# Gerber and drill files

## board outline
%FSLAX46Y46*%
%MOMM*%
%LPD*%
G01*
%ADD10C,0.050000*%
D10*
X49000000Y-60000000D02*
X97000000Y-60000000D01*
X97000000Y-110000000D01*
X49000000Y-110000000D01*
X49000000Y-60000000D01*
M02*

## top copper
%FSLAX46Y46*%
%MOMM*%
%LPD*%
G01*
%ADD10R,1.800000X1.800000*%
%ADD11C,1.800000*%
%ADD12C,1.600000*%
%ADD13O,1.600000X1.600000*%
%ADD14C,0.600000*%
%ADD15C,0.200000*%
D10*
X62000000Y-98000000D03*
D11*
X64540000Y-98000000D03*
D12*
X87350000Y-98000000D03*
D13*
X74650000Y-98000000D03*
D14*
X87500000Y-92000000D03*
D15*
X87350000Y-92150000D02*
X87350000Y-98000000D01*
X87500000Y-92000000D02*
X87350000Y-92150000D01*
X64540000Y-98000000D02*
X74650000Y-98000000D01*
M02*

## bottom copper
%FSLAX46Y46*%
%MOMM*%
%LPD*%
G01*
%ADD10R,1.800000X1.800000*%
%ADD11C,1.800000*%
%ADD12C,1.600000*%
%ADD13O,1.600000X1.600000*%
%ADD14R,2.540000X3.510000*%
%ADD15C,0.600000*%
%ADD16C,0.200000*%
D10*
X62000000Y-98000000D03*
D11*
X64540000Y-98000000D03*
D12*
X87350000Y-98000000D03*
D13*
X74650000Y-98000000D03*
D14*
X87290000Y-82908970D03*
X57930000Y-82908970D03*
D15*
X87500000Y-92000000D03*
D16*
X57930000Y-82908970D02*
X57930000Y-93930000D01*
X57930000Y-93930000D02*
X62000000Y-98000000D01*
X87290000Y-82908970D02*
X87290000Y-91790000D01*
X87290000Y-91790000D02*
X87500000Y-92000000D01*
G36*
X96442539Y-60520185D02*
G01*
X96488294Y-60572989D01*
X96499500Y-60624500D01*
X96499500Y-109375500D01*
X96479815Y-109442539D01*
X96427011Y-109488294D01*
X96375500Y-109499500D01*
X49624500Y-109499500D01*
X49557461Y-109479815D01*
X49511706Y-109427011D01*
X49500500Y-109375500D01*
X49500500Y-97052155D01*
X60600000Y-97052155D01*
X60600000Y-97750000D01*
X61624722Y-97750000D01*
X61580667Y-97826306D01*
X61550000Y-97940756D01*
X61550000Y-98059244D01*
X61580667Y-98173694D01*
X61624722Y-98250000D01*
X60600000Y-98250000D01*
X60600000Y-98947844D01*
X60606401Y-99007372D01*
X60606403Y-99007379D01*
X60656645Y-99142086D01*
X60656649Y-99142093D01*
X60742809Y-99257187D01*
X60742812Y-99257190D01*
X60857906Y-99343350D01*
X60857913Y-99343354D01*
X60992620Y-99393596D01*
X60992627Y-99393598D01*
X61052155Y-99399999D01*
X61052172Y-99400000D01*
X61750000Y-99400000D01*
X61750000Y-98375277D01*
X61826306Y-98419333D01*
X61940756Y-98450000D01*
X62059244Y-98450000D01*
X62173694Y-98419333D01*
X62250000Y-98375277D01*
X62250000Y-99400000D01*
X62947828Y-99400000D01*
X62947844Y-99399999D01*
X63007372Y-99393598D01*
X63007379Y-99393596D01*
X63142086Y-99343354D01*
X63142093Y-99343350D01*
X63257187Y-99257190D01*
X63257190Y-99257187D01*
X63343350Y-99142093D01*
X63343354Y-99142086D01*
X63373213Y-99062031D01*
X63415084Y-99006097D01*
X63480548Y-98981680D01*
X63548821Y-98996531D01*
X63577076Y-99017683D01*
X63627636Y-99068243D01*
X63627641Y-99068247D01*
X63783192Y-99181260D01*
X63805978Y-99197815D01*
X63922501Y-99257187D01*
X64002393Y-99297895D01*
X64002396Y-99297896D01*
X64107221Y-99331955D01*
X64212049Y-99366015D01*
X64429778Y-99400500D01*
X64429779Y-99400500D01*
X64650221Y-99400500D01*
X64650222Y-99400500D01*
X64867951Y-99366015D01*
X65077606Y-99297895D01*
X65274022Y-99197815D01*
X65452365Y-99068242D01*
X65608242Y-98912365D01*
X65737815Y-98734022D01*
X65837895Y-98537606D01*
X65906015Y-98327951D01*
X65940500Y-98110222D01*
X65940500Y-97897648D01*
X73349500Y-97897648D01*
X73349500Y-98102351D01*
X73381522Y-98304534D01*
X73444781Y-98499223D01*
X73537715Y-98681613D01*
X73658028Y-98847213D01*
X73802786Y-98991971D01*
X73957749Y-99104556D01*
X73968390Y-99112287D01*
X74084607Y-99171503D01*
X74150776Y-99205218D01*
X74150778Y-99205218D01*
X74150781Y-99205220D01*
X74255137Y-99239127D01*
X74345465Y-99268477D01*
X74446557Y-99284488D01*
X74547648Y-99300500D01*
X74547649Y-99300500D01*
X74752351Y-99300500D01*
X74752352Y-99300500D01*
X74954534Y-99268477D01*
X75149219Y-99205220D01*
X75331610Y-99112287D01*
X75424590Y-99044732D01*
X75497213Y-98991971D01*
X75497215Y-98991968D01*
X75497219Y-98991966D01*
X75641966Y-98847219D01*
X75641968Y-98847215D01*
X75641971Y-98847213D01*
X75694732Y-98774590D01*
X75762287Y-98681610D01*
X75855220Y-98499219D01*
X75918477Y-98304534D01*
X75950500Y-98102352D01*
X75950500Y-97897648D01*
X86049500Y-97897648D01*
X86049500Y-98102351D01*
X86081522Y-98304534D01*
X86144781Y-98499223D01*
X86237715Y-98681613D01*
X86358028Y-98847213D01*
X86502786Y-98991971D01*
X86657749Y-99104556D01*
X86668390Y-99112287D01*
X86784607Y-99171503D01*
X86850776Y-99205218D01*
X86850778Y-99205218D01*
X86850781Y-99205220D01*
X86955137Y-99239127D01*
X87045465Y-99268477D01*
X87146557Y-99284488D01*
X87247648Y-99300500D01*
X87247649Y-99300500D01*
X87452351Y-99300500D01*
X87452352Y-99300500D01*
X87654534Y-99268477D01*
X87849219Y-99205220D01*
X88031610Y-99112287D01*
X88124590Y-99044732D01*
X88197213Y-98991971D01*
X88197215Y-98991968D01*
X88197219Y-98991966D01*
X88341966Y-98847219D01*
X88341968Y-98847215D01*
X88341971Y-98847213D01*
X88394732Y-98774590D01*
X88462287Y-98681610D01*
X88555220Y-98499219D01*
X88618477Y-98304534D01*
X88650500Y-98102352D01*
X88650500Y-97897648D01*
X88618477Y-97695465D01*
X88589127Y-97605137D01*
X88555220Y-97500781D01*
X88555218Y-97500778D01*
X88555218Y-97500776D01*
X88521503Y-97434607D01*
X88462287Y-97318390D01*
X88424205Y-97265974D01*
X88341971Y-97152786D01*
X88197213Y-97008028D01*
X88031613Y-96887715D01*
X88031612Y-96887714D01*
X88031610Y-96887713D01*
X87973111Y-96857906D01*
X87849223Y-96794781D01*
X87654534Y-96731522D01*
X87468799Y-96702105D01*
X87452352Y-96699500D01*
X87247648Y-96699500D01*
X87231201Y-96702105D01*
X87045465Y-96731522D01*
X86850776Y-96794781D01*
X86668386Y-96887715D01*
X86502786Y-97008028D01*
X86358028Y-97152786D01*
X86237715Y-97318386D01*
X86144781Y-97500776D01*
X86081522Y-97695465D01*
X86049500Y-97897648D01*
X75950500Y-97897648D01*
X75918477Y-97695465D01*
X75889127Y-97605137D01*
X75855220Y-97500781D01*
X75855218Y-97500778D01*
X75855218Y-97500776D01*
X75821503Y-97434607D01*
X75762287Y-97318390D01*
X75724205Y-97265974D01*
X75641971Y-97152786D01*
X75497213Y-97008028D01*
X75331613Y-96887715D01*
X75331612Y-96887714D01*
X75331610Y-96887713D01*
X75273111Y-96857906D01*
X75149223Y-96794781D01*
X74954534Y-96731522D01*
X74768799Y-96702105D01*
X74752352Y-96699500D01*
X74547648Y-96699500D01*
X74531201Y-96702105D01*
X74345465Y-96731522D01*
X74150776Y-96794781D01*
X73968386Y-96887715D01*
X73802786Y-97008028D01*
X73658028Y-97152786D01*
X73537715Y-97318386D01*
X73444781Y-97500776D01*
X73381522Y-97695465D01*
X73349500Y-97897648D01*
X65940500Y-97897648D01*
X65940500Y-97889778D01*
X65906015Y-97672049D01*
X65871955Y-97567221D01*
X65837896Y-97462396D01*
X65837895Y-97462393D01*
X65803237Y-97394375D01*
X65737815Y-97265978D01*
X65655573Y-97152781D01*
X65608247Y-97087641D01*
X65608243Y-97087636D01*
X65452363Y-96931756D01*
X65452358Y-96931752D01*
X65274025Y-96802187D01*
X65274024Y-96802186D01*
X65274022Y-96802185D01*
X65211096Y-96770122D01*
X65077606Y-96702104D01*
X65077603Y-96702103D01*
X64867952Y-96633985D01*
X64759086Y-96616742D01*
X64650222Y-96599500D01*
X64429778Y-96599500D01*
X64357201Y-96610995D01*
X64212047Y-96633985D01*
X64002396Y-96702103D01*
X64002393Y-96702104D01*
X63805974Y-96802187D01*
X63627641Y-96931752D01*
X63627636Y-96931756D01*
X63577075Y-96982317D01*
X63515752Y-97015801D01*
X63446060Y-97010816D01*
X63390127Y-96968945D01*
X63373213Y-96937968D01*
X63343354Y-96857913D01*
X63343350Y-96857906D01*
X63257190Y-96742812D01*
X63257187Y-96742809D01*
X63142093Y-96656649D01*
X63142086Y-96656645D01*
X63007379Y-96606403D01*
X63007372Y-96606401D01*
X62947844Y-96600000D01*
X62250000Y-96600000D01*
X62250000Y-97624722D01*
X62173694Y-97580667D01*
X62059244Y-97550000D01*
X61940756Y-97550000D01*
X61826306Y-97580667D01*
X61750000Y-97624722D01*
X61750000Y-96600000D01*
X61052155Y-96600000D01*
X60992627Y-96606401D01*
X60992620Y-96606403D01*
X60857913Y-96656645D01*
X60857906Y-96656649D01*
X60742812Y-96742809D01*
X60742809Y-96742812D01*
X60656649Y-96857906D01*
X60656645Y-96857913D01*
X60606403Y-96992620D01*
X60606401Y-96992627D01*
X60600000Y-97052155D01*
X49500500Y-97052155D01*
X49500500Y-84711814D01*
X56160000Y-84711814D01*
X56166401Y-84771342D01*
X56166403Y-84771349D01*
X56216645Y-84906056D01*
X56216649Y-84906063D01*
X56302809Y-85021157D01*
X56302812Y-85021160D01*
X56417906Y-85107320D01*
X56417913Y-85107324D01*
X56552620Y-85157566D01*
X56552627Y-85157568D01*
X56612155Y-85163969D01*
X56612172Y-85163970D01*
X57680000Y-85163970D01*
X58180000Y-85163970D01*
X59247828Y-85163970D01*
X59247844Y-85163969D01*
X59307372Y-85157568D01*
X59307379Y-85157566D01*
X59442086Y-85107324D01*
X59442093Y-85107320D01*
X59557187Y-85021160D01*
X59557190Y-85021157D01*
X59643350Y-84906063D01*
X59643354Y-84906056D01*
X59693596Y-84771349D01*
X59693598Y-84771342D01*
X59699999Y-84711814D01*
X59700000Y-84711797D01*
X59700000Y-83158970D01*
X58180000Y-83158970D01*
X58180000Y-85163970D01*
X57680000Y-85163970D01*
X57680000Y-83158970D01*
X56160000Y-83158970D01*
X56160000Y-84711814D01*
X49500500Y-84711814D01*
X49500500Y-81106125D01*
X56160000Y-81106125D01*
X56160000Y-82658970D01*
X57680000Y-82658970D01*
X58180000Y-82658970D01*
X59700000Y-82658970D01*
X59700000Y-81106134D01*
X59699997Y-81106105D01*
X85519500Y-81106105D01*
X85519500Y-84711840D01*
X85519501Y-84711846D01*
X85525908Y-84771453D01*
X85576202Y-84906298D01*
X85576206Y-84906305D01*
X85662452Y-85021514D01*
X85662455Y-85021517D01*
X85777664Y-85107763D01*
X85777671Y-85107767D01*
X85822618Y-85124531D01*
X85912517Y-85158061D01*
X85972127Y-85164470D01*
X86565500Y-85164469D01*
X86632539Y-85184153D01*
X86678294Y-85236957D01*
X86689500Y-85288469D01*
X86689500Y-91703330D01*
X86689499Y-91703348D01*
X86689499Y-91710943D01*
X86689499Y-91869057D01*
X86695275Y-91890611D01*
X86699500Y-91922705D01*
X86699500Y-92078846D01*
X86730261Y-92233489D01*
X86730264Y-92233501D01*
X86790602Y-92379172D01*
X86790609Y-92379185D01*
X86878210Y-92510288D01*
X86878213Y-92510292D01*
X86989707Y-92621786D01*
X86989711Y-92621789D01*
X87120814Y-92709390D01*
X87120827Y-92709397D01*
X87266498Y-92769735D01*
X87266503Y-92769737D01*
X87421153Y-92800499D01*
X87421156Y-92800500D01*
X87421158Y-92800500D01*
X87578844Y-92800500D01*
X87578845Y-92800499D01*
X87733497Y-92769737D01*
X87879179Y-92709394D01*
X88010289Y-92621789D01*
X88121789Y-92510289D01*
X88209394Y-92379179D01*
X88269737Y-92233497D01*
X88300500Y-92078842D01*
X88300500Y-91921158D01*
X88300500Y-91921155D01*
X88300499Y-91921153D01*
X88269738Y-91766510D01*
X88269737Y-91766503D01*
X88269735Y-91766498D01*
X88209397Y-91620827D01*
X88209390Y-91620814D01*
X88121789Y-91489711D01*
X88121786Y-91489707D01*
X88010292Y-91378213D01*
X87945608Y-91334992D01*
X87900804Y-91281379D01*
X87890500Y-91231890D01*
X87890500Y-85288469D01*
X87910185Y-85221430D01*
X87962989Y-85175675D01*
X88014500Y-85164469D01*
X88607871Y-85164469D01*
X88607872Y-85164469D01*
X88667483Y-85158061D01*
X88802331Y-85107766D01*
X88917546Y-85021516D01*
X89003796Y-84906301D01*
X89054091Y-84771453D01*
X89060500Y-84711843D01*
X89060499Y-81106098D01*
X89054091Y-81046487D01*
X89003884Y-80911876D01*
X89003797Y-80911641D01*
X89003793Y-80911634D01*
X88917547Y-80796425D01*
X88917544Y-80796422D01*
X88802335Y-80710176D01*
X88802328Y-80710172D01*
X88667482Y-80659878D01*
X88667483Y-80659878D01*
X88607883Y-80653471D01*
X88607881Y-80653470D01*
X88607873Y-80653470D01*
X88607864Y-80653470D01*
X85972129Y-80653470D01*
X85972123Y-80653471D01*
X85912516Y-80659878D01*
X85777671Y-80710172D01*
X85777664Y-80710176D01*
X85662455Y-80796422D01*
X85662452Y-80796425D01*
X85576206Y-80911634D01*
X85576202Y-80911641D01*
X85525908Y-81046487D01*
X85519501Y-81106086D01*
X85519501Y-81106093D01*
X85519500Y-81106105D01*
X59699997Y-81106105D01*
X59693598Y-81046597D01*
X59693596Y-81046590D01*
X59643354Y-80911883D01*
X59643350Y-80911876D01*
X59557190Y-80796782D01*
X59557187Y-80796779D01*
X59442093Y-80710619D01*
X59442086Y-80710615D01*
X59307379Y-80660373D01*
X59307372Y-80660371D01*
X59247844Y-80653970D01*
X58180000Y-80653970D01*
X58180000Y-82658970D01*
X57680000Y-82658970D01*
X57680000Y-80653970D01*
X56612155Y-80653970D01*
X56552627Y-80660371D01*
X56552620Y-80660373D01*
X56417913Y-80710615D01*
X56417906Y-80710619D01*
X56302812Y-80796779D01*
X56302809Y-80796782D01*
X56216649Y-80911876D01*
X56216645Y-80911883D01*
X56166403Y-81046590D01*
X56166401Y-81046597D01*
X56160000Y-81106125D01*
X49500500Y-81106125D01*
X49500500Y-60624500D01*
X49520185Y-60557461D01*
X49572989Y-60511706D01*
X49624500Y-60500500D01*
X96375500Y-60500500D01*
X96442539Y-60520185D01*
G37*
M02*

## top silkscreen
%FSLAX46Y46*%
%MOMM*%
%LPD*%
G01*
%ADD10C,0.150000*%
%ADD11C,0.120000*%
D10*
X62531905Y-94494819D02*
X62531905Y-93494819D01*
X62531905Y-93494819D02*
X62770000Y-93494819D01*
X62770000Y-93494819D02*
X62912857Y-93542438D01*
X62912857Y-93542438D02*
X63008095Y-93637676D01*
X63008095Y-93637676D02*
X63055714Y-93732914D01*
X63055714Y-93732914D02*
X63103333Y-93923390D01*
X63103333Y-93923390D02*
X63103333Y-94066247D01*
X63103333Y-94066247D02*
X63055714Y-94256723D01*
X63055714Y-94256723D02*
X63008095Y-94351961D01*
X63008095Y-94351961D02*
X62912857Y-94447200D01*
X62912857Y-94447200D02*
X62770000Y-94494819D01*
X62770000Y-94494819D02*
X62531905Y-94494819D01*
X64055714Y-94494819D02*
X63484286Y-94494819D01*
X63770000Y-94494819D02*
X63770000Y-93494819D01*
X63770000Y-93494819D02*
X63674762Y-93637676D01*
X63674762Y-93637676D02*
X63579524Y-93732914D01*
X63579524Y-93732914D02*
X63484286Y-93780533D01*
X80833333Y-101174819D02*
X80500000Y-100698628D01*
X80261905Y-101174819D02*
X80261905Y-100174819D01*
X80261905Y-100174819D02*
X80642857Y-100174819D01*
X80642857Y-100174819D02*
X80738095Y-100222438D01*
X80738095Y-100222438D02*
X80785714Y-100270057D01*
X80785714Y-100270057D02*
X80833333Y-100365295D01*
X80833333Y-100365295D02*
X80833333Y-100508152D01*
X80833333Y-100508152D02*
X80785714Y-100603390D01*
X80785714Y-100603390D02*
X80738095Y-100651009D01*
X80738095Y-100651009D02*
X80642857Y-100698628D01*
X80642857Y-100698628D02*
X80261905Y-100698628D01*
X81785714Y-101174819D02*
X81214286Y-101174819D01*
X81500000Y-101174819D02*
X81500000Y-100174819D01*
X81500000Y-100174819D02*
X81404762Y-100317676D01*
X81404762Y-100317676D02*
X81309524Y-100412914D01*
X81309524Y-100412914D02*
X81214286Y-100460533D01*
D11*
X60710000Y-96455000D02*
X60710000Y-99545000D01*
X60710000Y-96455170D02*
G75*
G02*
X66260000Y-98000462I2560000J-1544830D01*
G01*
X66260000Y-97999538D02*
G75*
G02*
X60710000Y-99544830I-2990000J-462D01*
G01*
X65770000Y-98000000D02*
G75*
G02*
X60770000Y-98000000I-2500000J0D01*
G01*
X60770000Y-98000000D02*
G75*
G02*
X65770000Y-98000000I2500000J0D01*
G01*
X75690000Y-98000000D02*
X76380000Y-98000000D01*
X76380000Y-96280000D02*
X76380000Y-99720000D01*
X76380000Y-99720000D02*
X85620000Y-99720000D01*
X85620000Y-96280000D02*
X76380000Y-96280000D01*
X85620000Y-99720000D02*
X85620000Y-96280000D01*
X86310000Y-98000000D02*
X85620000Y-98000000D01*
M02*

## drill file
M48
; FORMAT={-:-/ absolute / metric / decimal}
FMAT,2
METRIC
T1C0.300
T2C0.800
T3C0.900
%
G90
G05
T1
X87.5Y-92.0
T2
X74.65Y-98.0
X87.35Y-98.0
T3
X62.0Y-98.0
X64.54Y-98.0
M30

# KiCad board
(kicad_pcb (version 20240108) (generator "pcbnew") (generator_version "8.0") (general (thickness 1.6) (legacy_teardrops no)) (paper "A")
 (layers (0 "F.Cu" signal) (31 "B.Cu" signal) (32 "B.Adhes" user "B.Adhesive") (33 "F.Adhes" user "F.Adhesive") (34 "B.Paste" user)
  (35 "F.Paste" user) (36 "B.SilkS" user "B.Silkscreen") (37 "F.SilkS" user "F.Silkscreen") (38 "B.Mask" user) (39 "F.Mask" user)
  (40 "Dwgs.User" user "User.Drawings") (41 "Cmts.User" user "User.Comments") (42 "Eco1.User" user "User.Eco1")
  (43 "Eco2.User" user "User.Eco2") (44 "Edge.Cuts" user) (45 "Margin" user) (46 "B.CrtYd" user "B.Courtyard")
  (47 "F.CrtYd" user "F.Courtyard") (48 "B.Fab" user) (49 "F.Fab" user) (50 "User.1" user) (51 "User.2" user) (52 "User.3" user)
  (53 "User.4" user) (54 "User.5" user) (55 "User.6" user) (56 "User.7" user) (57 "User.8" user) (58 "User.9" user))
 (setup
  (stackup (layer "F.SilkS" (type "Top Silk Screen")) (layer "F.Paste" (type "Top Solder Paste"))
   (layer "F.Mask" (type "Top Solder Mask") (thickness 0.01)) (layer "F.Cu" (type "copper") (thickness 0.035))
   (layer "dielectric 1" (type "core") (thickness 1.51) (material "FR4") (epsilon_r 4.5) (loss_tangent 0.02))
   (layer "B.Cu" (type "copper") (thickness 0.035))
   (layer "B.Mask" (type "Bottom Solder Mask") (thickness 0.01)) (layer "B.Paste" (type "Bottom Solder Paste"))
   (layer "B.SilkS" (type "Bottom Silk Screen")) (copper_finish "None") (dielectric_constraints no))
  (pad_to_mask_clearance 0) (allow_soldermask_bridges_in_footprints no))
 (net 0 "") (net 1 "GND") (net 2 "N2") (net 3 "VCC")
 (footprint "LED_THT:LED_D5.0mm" (layer "F.Cu") (at 62 98)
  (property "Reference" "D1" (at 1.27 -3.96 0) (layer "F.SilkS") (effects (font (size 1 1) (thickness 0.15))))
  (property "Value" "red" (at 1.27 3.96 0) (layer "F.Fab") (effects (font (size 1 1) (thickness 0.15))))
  (fp_line (start -1.29 -1.545) (end -1.29 1.545) (stroke (width 0.12) (type solid)) (layer "F.SilkS"))
  (fp_arc (start -1.29 -1.54483) (mid 2.072002 -2.880433) (end 4.26 0.000462) (stroke (width 0.12) (type solid)) (layer "F.SilkS"))
  (fp_arc (start 4.26 -0.000462) (mid 2.072002 2.880433) (end -1.29 1.54483) (stroke (width 0.12) (type solid)) (layer "F.SilkS"))
  (fp_circle (center 1.27 0) (end 3.77 0) (stroke (width 0.12) (type solid)) (fill none) (layer "F.SilkS"))
  (pad "1" thru_hole rect (at 0 0) (size 1.8 1.8) (drill 0.9) (layers "*.Cu" "*.Mask") (remove_unused_layers no) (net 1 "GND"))
  (pad "2" thru_hole circle (at 2.54 0) (size 1.8 1.8) (drill 0.9) (layers "*.Cu" "*.Mask") (remove_unused_layers no) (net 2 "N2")))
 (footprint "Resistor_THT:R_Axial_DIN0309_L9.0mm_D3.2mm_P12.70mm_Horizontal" (layer "F.Cu") (at 87.35 98 180)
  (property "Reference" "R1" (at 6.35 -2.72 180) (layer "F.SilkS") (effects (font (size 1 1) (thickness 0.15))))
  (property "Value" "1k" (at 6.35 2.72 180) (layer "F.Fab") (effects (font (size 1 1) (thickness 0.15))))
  (fp_line (start 11.66 0) (end 10.97 0) (stroke (width 0.12) (type solid)) (layer "F.SilkS"))
  (fp_line (start 10.97 1.72) (end 10.97 -1.72) (stroke (width 0.12) (type solid)) (layer "F.SilkS"))
  (fp_line (start 10.97 -1.72) (end 1.73 -1.72) (stroke (width 0.12) (type solid)) (layer "F.SilkS"))
  (fp_line (start 1.73 1.72) (end 10.97 1.72) (stroke (width 0.12) (type solid)) (layer "F.SilkS"))
  (fp_line (start 1.73 -1.72) (end 1.73 1.72) (stroke (width 0.12) (type solid)) (layer "F.SilkS"))
  (fp_line (start 1.04 0) (end 1.73 0) (stroke (width 0.12) (type solid)) (layer "F.SilkS"))
  (pad "1" thru_hole circle (at 0 0 180) (size 1.6 1.6) (drill 0.8) (layers "*.Cu" "*.Mask") (remove_unused_layers no) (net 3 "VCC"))
  (pad "2" thru_hole oval (at 12.7 0 180) (size 1.6 1.6) (drill 0.8) (layers "*.Cu" "*.Mask") (remove_unused_layers no) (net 2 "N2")))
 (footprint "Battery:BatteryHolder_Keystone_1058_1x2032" (layer "B.Cu") (at 72.61 82.90897 180)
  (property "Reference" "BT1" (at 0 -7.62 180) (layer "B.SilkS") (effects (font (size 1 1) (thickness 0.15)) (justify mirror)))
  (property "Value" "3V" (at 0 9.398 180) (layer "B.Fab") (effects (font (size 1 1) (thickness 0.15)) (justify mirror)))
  (pad "1" smd rect (at -14.68 0 180) (size 2.54 3.51) (layers "B.Cu" "B.Paste" "B.Mask") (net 3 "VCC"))
  (pad "2" smd rect (at 14.68 0 180) (size 2.54 3.51) (layers "B.Cu" "B.Paste" "B.Mask") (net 1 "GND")))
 (gr_rect (start 49 60) (end 97 110) (stroke (width 0.05) (type default)) (fill none) (layer "Edge.Cuts"))
 (segment (start 57.93 82.90897) (end 57.93 93.93) (width 0.2) (layer "B.Cu") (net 1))
 (segment (start 57.93 93.93) (end 62 98) (width 0.2) (layer "B.Cu") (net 1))
 (segment (start 87.35 92.15) (end 87.35 98) (width 0.2) (layer "F.Cu") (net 3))
 (segment (start 87.5 92) (end 87.35 92.15) (width 0.2) (layer "F.Cu") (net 3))
 (via (at 87.5 92) (size 0.6) (drill 0.3) (layers "F.Cu" "B.Cu") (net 3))
 (segment (start 87.29 82.90897) (end 87.29 91.79) (width 0.2) (layer "B.Cu") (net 3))
 (segment (start 87.29 91.79) (end 87.5 92) (width 0.2) (layer "B.Cu") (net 3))
 (segment (start 64.54 98) (end 74.65 98) (width 0.2) (layer "F.Cu") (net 2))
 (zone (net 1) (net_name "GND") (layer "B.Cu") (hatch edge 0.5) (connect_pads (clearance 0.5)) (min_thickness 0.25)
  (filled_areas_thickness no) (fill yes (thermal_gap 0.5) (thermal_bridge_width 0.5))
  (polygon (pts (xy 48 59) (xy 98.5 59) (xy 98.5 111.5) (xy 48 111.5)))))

